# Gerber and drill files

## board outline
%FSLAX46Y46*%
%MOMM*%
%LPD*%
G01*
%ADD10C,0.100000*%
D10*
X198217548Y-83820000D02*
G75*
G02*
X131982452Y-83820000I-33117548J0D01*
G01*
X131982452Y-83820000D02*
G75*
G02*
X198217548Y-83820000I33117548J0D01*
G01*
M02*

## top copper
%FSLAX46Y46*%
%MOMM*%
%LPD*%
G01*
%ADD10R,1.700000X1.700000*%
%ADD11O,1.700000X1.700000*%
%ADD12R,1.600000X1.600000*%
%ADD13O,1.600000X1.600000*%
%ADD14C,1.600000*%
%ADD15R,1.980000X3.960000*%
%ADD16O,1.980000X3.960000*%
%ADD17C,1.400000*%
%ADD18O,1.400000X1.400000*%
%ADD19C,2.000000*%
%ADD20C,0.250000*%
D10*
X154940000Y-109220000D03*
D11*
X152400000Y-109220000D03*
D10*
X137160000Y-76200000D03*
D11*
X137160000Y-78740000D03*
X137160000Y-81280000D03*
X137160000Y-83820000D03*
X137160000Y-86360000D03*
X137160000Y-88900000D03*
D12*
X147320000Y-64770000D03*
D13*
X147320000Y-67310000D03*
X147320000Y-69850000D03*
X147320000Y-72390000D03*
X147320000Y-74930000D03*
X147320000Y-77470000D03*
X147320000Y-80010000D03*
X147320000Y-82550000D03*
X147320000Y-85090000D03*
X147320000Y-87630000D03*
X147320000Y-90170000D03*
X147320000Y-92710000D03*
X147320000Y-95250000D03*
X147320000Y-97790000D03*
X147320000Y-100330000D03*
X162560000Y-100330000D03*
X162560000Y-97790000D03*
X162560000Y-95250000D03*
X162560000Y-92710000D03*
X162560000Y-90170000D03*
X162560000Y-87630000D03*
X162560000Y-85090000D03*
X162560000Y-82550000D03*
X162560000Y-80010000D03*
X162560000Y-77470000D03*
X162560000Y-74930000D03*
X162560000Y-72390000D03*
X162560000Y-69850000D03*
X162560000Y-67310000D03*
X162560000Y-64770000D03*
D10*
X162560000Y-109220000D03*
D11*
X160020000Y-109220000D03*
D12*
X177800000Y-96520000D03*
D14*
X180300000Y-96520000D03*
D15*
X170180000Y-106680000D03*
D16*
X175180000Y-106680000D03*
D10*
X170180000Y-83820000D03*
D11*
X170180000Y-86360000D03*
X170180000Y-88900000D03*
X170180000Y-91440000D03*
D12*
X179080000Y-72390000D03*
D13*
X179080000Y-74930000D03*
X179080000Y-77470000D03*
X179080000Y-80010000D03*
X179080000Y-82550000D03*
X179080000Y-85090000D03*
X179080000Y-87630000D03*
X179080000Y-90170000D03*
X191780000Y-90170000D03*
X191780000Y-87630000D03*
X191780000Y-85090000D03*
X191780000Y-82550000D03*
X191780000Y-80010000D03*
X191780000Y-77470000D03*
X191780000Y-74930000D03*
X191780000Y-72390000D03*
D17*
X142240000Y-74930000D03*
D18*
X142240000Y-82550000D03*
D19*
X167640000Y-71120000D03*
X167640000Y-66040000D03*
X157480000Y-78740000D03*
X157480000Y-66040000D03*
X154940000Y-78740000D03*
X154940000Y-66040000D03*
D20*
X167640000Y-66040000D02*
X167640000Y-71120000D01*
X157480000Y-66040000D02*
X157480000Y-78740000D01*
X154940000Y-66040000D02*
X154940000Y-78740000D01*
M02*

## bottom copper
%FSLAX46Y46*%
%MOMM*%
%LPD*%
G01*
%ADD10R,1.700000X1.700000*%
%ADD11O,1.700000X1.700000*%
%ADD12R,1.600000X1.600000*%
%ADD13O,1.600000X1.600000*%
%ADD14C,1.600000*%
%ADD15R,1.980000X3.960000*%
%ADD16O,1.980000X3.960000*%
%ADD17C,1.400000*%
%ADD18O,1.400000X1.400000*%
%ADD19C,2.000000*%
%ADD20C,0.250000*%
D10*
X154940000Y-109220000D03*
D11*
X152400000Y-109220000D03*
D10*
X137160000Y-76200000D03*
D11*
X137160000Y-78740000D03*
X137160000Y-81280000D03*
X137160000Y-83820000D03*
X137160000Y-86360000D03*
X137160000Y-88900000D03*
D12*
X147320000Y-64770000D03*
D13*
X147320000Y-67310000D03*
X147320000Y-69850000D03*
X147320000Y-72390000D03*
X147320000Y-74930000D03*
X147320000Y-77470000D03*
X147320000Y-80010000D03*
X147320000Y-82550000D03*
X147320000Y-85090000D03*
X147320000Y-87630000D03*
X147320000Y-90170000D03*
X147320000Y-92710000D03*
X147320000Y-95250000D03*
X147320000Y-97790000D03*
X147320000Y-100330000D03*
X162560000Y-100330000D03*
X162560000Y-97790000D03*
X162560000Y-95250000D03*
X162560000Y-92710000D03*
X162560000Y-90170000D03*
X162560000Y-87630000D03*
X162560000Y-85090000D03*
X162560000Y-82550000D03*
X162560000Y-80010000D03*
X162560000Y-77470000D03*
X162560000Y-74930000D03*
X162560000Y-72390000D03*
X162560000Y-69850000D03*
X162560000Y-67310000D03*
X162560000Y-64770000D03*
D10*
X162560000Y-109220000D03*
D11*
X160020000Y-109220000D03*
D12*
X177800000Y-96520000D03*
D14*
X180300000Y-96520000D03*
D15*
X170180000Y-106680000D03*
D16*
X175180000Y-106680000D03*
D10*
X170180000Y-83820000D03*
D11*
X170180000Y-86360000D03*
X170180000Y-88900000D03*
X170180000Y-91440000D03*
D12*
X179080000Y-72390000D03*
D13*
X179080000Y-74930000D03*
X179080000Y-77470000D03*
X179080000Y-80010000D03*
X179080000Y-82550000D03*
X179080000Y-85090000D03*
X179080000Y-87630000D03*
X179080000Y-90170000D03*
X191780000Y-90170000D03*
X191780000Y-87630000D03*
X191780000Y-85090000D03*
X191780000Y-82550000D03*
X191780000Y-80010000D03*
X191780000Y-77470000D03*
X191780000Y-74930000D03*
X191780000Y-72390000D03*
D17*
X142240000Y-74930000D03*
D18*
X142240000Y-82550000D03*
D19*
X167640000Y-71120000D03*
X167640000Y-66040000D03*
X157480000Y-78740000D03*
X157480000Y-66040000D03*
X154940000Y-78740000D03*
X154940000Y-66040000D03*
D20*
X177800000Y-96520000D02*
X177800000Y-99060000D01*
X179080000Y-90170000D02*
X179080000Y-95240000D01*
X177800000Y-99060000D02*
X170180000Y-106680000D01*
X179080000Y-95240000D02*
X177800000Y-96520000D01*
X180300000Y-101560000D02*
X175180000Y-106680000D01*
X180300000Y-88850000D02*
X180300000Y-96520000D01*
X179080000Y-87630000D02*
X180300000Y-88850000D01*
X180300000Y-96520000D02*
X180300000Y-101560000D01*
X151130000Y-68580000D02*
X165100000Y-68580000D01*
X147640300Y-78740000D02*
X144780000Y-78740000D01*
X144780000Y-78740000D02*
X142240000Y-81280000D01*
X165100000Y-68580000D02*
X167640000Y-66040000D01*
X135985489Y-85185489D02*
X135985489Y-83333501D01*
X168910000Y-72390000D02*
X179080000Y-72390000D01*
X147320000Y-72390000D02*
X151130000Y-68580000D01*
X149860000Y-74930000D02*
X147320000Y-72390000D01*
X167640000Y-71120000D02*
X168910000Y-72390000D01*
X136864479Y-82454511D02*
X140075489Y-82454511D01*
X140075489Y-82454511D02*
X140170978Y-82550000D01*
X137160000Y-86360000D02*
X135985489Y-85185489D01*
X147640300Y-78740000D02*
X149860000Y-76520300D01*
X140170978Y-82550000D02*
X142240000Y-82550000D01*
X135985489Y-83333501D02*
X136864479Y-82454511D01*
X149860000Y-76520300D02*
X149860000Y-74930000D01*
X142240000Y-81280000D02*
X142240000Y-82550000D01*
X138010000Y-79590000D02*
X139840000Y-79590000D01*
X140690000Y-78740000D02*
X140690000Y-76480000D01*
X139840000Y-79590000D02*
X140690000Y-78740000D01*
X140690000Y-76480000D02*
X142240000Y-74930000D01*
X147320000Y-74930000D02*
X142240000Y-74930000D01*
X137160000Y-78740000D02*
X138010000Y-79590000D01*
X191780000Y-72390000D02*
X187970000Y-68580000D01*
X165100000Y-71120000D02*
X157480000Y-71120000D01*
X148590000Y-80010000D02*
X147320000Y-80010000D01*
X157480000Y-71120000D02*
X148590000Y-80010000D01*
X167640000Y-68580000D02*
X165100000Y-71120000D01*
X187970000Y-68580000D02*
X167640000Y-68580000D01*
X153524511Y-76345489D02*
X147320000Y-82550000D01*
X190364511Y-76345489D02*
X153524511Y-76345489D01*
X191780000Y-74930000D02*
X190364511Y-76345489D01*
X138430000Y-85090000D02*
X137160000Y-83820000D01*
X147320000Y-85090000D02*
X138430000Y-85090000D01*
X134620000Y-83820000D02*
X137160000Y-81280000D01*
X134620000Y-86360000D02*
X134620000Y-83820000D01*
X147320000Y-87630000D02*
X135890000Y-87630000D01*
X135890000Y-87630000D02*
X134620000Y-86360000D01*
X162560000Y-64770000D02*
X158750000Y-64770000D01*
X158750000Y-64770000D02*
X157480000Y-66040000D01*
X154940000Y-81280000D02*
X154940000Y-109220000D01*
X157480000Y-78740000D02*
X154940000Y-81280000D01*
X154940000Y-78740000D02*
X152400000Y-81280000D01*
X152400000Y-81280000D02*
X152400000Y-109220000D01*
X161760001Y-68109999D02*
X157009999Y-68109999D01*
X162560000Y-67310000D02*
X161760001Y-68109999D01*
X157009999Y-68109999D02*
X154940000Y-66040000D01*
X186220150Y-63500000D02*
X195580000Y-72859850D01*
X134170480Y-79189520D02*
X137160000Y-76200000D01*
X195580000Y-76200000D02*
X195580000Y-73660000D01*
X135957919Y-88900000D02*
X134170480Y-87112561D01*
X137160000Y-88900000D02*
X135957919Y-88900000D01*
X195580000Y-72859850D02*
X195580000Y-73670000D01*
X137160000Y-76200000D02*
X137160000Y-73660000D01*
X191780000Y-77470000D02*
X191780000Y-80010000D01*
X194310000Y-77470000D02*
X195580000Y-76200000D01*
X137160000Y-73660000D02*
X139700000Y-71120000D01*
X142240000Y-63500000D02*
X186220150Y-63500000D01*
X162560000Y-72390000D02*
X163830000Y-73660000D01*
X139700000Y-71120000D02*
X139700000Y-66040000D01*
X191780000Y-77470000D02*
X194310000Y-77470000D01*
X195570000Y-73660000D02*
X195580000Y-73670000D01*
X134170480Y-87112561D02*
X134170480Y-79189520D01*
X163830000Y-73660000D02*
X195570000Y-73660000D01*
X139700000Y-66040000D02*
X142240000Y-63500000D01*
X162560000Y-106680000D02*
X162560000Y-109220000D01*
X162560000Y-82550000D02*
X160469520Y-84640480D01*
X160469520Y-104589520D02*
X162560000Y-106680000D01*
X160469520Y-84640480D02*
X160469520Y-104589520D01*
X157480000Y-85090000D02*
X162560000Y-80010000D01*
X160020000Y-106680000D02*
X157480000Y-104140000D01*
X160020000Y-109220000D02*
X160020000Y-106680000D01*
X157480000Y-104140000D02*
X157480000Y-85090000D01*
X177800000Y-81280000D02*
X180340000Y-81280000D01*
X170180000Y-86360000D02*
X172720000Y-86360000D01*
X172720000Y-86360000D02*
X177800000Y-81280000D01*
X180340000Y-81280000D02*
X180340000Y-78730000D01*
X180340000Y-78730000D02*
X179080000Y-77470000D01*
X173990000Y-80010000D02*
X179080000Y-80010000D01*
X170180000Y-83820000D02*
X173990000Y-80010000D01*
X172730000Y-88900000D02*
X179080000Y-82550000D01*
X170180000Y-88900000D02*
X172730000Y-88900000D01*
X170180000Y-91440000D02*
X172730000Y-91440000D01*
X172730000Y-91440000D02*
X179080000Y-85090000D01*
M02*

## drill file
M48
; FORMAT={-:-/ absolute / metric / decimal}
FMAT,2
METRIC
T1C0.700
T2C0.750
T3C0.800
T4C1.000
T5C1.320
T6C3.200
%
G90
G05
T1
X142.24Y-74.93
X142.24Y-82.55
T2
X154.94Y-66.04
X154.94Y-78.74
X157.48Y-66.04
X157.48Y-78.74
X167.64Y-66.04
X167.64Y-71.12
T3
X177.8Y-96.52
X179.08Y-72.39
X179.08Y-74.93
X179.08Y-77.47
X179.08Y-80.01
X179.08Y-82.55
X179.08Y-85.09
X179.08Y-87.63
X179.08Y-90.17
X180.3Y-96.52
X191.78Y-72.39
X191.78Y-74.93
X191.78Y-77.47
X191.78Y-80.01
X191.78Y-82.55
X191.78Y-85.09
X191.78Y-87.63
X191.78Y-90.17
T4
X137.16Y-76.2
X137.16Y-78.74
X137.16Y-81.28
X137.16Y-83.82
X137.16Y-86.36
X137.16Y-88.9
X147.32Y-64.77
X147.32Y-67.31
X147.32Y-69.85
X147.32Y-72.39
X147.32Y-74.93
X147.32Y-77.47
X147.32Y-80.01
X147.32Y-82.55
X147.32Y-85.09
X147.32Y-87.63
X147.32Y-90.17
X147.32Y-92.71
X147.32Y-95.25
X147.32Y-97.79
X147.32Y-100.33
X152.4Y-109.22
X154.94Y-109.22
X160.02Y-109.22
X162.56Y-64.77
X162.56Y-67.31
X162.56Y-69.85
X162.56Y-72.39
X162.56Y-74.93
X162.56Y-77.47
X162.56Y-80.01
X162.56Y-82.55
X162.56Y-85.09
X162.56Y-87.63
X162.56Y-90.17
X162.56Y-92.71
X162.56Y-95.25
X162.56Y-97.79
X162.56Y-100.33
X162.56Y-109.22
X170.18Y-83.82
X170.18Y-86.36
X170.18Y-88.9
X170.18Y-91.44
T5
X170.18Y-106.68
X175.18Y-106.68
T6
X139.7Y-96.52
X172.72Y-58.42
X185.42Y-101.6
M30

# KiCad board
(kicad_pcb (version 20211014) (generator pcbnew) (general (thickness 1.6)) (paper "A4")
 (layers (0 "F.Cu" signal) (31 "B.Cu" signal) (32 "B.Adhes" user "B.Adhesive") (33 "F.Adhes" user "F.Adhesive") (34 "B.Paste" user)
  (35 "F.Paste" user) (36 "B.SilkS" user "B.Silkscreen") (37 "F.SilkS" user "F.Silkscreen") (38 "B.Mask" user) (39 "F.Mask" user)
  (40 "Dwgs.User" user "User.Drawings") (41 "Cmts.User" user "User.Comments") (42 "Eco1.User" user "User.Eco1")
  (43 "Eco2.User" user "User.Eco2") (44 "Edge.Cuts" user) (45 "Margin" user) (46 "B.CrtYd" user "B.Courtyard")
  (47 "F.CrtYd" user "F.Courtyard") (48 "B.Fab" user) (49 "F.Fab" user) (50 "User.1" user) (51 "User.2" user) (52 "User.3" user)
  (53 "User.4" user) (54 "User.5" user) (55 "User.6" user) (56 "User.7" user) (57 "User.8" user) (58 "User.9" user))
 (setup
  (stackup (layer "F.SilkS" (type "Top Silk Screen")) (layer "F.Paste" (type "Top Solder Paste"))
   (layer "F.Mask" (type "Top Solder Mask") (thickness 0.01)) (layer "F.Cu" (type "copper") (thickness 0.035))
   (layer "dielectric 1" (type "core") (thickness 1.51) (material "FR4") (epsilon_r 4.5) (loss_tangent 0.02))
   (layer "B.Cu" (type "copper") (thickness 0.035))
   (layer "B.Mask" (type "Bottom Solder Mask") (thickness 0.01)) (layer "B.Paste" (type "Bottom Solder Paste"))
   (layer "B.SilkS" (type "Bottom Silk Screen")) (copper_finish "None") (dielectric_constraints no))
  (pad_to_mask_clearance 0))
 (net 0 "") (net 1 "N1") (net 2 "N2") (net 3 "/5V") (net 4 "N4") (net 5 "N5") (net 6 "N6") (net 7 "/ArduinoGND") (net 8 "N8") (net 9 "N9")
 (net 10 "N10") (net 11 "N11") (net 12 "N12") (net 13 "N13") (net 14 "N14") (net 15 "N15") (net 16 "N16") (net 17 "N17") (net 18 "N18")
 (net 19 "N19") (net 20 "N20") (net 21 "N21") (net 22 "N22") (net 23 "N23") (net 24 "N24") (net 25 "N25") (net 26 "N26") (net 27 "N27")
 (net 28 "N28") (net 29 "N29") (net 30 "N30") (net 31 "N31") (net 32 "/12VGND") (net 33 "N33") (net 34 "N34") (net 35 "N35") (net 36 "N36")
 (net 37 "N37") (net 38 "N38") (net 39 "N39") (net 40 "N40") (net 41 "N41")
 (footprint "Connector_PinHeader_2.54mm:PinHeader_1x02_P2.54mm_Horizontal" (layer "F.Cu") (at 154.94 109.22 -90)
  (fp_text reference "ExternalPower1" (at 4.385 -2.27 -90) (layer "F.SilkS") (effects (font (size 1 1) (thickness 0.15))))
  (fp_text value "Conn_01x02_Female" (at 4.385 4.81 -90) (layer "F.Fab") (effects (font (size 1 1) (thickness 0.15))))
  (pad "1" thru_hole rect (at 0 0 270) (size 1.7 1.7) (drill 1) (layers *.Cu *.Mask) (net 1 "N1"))
  (pad "2" thru_hole oval (at 0 2.54 270) (size 1.7 1.7) (drill 1) (layers *.Cu *.Mask) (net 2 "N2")))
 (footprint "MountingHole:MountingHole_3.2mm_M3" (layer "F.Cu") (at 139.7 96.52)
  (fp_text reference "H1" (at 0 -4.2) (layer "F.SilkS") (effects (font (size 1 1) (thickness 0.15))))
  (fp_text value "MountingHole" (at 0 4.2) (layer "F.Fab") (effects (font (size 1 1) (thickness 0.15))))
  (pad "" np_thru_hole circle (at 0 0) (size 3.2 3.2) (drill 3.2) (layers *.Cu *.Mask)))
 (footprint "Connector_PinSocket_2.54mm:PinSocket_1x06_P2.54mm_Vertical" (layer "F.Cu") (at 137.16 76.2)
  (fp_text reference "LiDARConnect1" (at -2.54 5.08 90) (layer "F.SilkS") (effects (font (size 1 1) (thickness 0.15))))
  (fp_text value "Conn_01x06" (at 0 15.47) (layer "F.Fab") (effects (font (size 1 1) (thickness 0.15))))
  (pad "1" thru_hole rect (at 0 0) (size 1.7 1.7) (drill 1) (layers *.Cu *.Mask) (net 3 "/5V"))
  (pad "2" thru_hole oval (at 0 2.54) (size 1.7 1.7) (drill 1) (layers *.Cu *.Mask) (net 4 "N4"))
  (pad "3" thru_hole oval (at 0 5.08) (size 1.7 1.7) (drill 1) (layers *.Cu *.Mask) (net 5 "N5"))
  (pad "4" thru_hole oval (at 0 7.62) (size 1.7 1.7) (drill 1) (layers *.Cu *.Mask) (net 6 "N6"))
  (pad "5" thru_hole oval (at 0 10.16) (size 1.7 1.7) (drill 1) (layers *.Cu *.Mask) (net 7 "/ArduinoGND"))
  (pad "6" thru_hole oval (at 0 12.7) (size 1.7 1.7) (drill 1) (layers *.Cu *.Mask) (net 3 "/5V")))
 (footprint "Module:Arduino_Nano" (layer "F.Cu") (at 147.32 64.77)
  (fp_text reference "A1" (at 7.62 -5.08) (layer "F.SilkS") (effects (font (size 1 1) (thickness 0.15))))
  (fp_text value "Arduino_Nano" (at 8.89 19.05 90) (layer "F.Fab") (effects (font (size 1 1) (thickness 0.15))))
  (pad "1" thru_hole rect (at 0 0) (size 1.6 1.6) (drill 1) (layers *.Cu *.Mask) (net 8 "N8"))
  (pad "2" thru_hole oval (at 0 2.54) (size 1.6 1.6) (drill 1) (layers *.Cu *.Mask) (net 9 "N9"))
  (pad "3" thru_hole oval (at 0 5.08) (size 1.6 1.6) (drill 1) (layers *.Cu *.Mask) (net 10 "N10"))
  (pad "4" thru_hole oval (at 0 7.62) (size 1.6 1.6) (drill 1) (layers *.Cu *.Mask) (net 7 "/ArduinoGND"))
  (pad "5" thru_hole oval (at 0 10.16) (size 1.6 1.6) (drill 1) (layers *.Cu *.Mask) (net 4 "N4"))
  (pad "6" thru_hole oval (at 0 12.7) (size 1.6 1.6) (drill 1) (layers *.Cu *.Mask) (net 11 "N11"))
  (pad "7" thru_hole oval (at 0 15.24) (size 1.6 1.6) (drill 1) (layers *.Cu *.Mask) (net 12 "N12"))
  (pad "8" thru_hole oval (at 0 17.78) (size 1.6 1.6) (drill 1) (layers *.Cu *.Mask) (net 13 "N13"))
  (pad "9" thru_hole oval (at 0 20.32) (size 1.6 1.6) (drill 1) (layers *.Cu *.Mask) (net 6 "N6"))
  (pad "10" thru_hole oval (at 0 22.86) (size 1.6 1.6) (drill 1) (layers *.Cu *.Mask) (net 5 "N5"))
  (pad "11" thru_hole oval (at 0 25.4) (size 1.6 1.6) (drill 1) (layers *.Cu *.Mask) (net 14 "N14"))
  (pad "12" thru_hole oval (at 0 27.94) (size 1.6 1.6) (drill 1) (layers *.Cu *.Mask) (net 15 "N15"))
  (pad "13" thru_hole oval (at 0 30.48) (size 1.6 1.6) (drill 1) (layers *.Cu *.Mask) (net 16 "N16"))
  (pad "14" thru_hole oval (at 0 33.02) (size 1.6 1.6) (drill 1) (layers *.Cu *.Mask) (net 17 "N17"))
  (pad "15" thru_hole oval (at 0 35.56) (size 1.6 1.6) (drill 1) (layers *.Cu *.Mask) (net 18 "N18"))
  (pad "16" thru_hole oval (at 15.24 35.56) (size 1.6 1.6) (drill 1) (layers *.Cu *.Mask) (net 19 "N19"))
  (pad "17" thru_hole oval (at 15.24 33.02) (size 1.6 1.6) (drill 1) (layers *.Cu *.Mask) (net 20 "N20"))
  (pad "18" thru_hole oval (at 15.24 30.48) (size 1.6 1.6) (drill 1) (layers *.Cu *.Mask) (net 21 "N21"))
  (pad "19" thru_hole oval (at 15.24 27.94) (size 1.6 1.6) (drill 1) (layers *.Cu *.Mask) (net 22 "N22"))
  (pad "20" thru_hole oval (at 15.24 25.4) (size 1.6 1.6) (drill 1) (layers *.Cu *.Mask) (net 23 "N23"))
  (pad "21" thru_hole oval (at 15.24 22.86) (size 1.6 1.6) (drill 1) (layers *.Cu *.Mask) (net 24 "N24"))
  (pad "22" thru_hole oval (at 15.24 20.32) (size 1.6 1.6) (drill 1) (layers *.Cu *.Mask) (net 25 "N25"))
  (pad "23" thru_hole oval (at 15.24 17.78) (size 1.6 1.6) (drill 1) (layers *.Cu *.Mask) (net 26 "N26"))
  (pad "24" thru_hole oval (at 15.24 15.24) (size 1.6 1.6) (drill 1) (layers *.Cu *.Mask) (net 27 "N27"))
  (pad "25" thru_hole oval (at 15.24 12.7) (size 1.6 1.6) (drill 1) (layers *.Cu *.Mask) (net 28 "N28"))
  (pad "26" thru_hole oval (at 15.24 10.16) (size 1.6 1.6) (drill 1) (layers *.Cu *.Mask) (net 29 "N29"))
  (pad "27" thru_hole oval (at 15.24 7.62) (size 1.6 1.6) (drill 1) (layers *.Cu *.Mask) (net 3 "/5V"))
  (pad "28" thru_hole oval (at 15.24 5.08) (size 1.6 1.6) (drill 1) (layers *.Cu *.Mask) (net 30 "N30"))
  (pad "29" thru_hole oval (at 15.24 2.54) (size 1.6 1.6) (drill 1) (layers *.Cu *.Mask) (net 2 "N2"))
  (pad "30" thru_hole oval (at 15.24 0) (size 1.6 1.6) (drill 1) (layers *.Cu *.Mask) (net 1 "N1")))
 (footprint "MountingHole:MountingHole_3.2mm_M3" (layer "F.Cu") (at 185.42 101.6)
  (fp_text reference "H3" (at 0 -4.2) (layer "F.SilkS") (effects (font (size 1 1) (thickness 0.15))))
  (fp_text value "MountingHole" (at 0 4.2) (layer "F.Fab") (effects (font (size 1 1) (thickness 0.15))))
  (pad "" np_thru_hole circle (at 0 0) (size 3.2 3.2) (drill 3.2) (layers *.Cu *.Mask)))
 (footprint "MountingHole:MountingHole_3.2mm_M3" (layer "F.Cu") (at 172.72 58.42)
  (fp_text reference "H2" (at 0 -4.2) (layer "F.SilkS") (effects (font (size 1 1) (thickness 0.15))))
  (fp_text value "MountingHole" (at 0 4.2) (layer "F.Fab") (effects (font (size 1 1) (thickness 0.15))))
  (pad "" np_thru_hole circle (at 0 0) (size 3.2 3.2) (drill 3.2) (layers *.Cu *.Mask)))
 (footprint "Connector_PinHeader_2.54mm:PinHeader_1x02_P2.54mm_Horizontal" (layer "F.Cu") (at 162.56 109.22 -90)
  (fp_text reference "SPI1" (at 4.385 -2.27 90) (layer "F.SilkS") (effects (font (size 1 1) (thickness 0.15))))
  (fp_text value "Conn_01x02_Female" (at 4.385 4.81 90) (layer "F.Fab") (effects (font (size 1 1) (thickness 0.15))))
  (pad "1" thru_hole rect (at 0 0 270) (size 1.7 1.7) (drill 1) (layers *.Cu *.Mask) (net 26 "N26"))
  (pad "2" thru_hole oval (at 0 2.54 270) (size 1.7 1.7) (drill 1) (layers *.Cu *.Mask) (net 27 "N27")))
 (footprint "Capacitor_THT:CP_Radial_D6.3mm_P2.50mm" (layer "F.Cu") (at 177.8 96.52)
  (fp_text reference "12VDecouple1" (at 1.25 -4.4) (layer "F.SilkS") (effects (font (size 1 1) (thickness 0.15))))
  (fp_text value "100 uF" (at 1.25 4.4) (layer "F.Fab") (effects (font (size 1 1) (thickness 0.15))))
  (pad "1" thru_hole rect (at 0 0) (size 1.6 1.6) (drill 0.8) (layers *.Cu *.Mask) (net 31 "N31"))
  (pad "2" thru_hole circle (at 2.5 0) (size 1.6 1.6) (drill 0.8) (layers *.Cu *.Mask) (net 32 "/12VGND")))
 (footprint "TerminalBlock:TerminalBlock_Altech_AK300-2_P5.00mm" (layer "F.Cu") (at 170.18 106.68)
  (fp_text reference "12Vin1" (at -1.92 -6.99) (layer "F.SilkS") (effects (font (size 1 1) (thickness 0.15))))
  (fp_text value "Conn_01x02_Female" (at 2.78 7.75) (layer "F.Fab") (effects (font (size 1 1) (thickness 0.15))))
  (pad "1" thru_hole rect (at 0 0) (size 1.98 3.96) (drill 1.32) (layers *.Cu *.Mask) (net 31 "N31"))
  (pad "2" thru_hole oval (at 5 0) (size 1.98 3.96) (drill 1.32) (layers *.Cu *.Mask) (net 32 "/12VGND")))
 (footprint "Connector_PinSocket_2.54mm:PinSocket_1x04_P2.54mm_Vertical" (layer "F.Cu") (at 170.18 83.82)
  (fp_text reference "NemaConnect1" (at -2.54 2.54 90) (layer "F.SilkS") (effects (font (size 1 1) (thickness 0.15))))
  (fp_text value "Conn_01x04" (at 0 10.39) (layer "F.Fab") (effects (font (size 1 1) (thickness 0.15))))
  (pad "1" thru_hole rect (at 0 0) (size 1.7 1.7) (drill 1) (layers *.Cu *.Mask) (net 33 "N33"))
  (pad "2" thru_hole oval (at 0 2.54) (size 1.7 1.7) (drill 1) (layers *.Cu *.Mask) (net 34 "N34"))
  (pad "3" thru_hole oval (at 0 5.08) (size 1.7 1.7) (drill 1) (layers *.Cu *.Mask) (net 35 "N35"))
  (pad "4" thru_hole oval (at 0 7.62) (size 1.7 1.7) (drill 1) (layers *.Cu *.Mask) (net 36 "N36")))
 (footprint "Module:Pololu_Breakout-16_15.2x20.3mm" (layer "F.Cu") (at 179.08 72.39)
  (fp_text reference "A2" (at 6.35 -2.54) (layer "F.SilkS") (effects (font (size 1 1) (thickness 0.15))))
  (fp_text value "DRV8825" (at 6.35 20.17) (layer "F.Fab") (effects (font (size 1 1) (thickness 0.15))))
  (pad "1" thru_hole rect (at 0 0) (size 1.6 1.6) (drill 0.8) (layers *.Cu *.Mask) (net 7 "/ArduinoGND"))
  (pad "2" thru_hole oval (at 0 2.54) (size 1.6 1.6) (drill 0.8) (layers *.Cu *.Mask) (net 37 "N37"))
  (pad "3" thru_hole oval (at 0 5.08) (size 1.6 1.6) (drill 0.8) (layers *.Cu *.Mask) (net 34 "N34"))
  (pad "4" thru_hole oval (at 0 7.62) (size 1.6 1.6) (drill 0.8) (layers *.Cu *.Mask) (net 33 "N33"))
  (pad "5" thru_hole oval (at 0 10.16) (size 1.6 1.6) (drill 0.8) (layers *.Cu *.Mask) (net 35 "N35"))
  (pad "6" thru_hole oval (at 0 12.7) (size 1.6 1.6) (drill 0.8) (layers *.Cu *.Mask) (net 36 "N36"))
  (pad "7" thru_hole oval (at 0 15.24) (size 1.6 1.6) (drill 0.8) (layers *.Cu *.Mask) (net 32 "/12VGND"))
  (pad "8" thru_hole oval (at 0 17.78) (size 1.6 1.6) (drill 0.8) (layers *.Cu *.Mask) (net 31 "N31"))
  (pad "9" thru_hole oval (at 12.7 17.78) (size 1.6 1.6) (drill 0.8) (layers *.Cu *.Mask) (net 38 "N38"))
  (pad "10" thru_hole oval (at 12.7 15.24) (size 1.6 1.6) (drill 0.8) (layers *.Cu *.Mask) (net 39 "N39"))
  (pad "11" thru_hole oval (at 12.7 12.7) (size 1.6 1.6) (drill 0.8) (layers *.Cu *.Mask) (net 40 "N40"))
  (pad "12" thru_hole oval (at 12.7 10.16) (size 1.6 1.6) (drill 0.8) (layers *.Cu *.Mask) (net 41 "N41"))
  (pad "13" thru_hole oval (at 12.7 7.62) (size 1.6 1.6) (drill 0.8) (layers *.Cu *.Mask) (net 3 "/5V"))
  (pad "14" thru_hole oval (at 12.7 5.08) (size 1.6 1.6) (drill 0.8) (layers *.Cu *.Mask) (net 3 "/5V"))
  (pad "15" thru_hole oval (at 12.7 2.54) (size 1.6 1.6) (drill 0.8) (layers *.Cu *.Mask) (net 13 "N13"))
  (pad "16" thru_hole oval (at 12.7 0) (size 1.6 1.6) (drill 0.8) (layers *.Cu *.Mask) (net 12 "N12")))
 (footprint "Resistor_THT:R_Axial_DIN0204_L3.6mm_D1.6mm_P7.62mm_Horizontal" (layer "B.Cu") (at 142.24 74.93 -90)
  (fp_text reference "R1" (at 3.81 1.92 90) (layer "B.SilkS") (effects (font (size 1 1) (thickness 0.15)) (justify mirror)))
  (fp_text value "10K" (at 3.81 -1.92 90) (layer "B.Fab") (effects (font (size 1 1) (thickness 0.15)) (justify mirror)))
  (pad "1" thru_hole circle (at 0 0 270) (size 1.4 1.4) (drill 0.7) (layers *.Cu *.Mask) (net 4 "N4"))
  (pad "2" thru_hole oval (at 7.62 0 270) (size 1.4 1.4) (drill 0.7) (layers *.Cu *.Mask) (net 7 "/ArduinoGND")))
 (gr_circle (center 165.1 83.82) (end 193.04 66.04) (layer "Edge.Cuts") (width 0.1) (fill none))
 (segment (start 177.8 96.52) (end 177.8 99.06) (width 0.25) (layer "B.Cu") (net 31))
 (segment (start 179.08 90.17) (end 179.08 95.24) (width 0.25) (layer "B.Cu") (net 31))
 (segment (start 177.8 99.06) (end 170.18 106.68) (width 0.25) (layer "B.Cu") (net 31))
 (segment (start 179.08 95.24) (end 177.8 96.52) (width 0.25) (layer "B.Cu") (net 31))
 (segment (start 180.3 101.56) (end 175.18 106.68) (width 0.25) (layer "B.Cu") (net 32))
 (segment (start 180.3 88.85) (end 180.3 96.52) (width 0.25) (layer "B.Cu") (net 32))
 (segment (start 179.08 87.63) (end 180.3 88.85) (width 0.25) (layer "B.Cu") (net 32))
 (segment (start 180.3 96.52) (end 180.3 101.56) (width 0.25) (layer "B.Cu") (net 32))
 (segment (start 167.64 66.04) (end 167.64 71.12) (width 0.25) (layer "F.Cu") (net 7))
 (via (at 167.64 71.12) (size 2) (drill 0.75) (layers "F.Cu" "B.Cu") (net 7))
 (via (at 167.64 66.04) (size 2) (drill 0.75) (layers "F.Cu" "B.Cu") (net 7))
 (segment (start 151.13 68.58) (end 165.1 68.58) (width 0.25) (layer "B.Cu") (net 7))
 (segment (start 147.6403 78.74) (end 144.78 78.74) (width 0.25) (layer "B.Cu") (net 7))
 (segment (start 144.78 78.74) (end 142.24 81.28) (width 0.25) (layer "B.Cu") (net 7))
 (segment (start 165.1 68.58) (end 167.64 66.04) (width 0.25) (layer "B.Cu") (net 7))
 (segment (start 135.985489 85.185489) (end 135.985489 83.333501) (width 0.25) (layer "B.Cu") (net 7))
 (segment (start 168.91 72.39) (end 179.08 72.39) (width 0.25) (layer "B.Cu") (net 7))
 (segment (start 147.32 72.39) (end 151.13 68.58) (width 0.25) (layer "B.Cu") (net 7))
 (segment (start 149.86 74.93) (end 147.32 72.39) (width 0.25) (layer "B.Cu") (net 7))
 (segment (start 167.64 71.12) (end 168.91 72.39) (width 0.25) (layer "B.Cu") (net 7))
 (segment (start 136.864479 82.454511) (end 140.075489 82.454511) (width 0.25) (layer "B.Cu") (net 7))
 (segment (start 140.075489 82.454511) (end 140.170978 82.55) (width 0.25) (layer "B.Cu") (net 7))
 (segment (start 137.16 86.36) (end 135.985489 85.185489) (width 0.25) (layer "B.Cu") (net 7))
 (segment (start 147.6403 78.74) (end 149.86 76.5203) (width 0.25) (layer "B.Cu") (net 7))
 (segment (start 140.170978 82.55) (end 142.24 82.55) (width 0.25) (layer "B.Cu") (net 7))
 (segment (start 135.985489 83.333501) (end 136.864479 82.454511) (width 0.25) (layer "B.Cu") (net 7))
 (segment (start 149.86 76.5203) (end 149.86 74.93) (width 0.25) (layer "B.Cu") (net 7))
 (segment (start 142.24 81.28) (end 142.24 82.55) (width 0.25) (layer "B.Cu") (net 7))
 (segment (start 138.01 79.59) (end 139.84 79.59) (width 0.25) (layer "B.Cu") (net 4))
 (segment (start 140.69 78.74) (end 140.69 76.48) (width 0.25) (layer "B.Cu") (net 4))
 (segment (start 139.84 79.59) (end 140.69 78.74) (width 0.25) (layer "B.Cu") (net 4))
 (segment (start 140.69 76.48) (end 142.24 74.93) (width 0.25) (layer "B.Cu") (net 4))
 (segment (start 147.32 74.93) (end 142.24 74.93) (width 0.25) (layer "B.Cu") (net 4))
 (segment (start 137.16 78.74) (end 138.01 79.59) (width 0.25) (layer "B.Cu") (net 4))
 (segment (start 191.78 72.39) (end 187.97 68.58) (width 0.25) (layer "B.Cu") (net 12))
 (segment (start 165.1 71.12) (end 157.48 71.12) (width 0.25) (layer "B.Cu") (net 12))
 (segment (start 148.59 80.01) (end 147.32 80.01) (width 0.25) (layer "B.Cu") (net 12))
 (segment (start 157.48 71.12) (end 148.59 80.01) (width 0.25) (layer "B.Cu") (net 12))
 (segment (start 167.64 68.58) (end 165.1 71.12) (width 0.25) (layer "B.Cu") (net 12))
 (segment (start 187.97 68.58) (end 167.64 68.58) (width 0.25) (layer "B.Cu") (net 12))
 (segment (start 153.524511 76.345489) (end 147.32 82.55) (width 0.25) (layer "B.Cu") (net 13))
 (segment (start 190.364511 76.345489) (end 153.524511 76.345489) (width 0.25) (layer "B.Cu") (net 13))
 (segment (start 191.78 74.93) (end 190.364511 76.345489) (width 0.25) (layer "B.Cu") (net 13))
 (segment (start 138.43 85.09) (end 137.16 83.82) (width 0.25) (layer "B.Cu") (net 6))
 (segment (start 147.32 85.09) (end 138.43 85.09) (width 0.25) (layer "B.Cu") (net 6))
 (segment (start 134.62 83.82) (end 137.16 81.28) (width 0.25) (layer "B.Cu") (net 5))
 (segment (start 134.62 86.36) (end 134.62 83.82) (width 0.25) (layer "B.Cu") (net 5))
 (segment (start 147.32 87.63) (end 135.89 87.63) (width 0.25) (layer "B.Cu") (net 5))
 (segment (start 135.89 87.63) (end 134.62 86.36) (width 0.25) (layer "B.Cu") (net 5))
 (segment (start 157.48 66.04) (end 157.48 78.74) (width 0.25) (layer "F.Cu") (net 1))
 (via (at 157.48 78.74) (size 2) (drill 0.75) (layers "F.Cu" "B.Cu") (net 1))
 (via (at 157.48 66.04) (size 2) (drill 0.75) (layers "F.Cu" "B.Cu") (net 1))
 (segment (start 162.56 64.77) (end 158.75 64.77) (width 0.25) (layer "B.Cu") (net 1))
 (segment (start 158.75 64.77) (end 157.48 66.04) (width 0.25) (layer "B.Cu") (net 1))
 (segment (start 154.94 81.28) (end 154.94 109.22) (width 0.25) (layer "B.Cu") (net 1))
 (segment (start 157.48 78.74) (end 154.94 81.28) (width 0.25) (layer "B.Cu") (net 1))
 (segment (start 154.94 66.04) (end 154.94 78.74) (width 0.25) (layer "F.Cu") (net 2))
 (via (at 154.94 78.74) (size 2) (drill 0.75) (layers "F.Cu" "B.Cu") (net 2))
 (via (at 154.94 66.04) (size 2) (drill 0.75) (layers "F.Cu" "B.Cu") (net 2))
 (segment (start 154.94 78.74) (end 152.4 81.28) (width 0.25) (layer "B.Cu") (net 2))
 (segment (start 152.4 81.28) (end 152.4 109.22) (width 0.25) (layer "B.Cu") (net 2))
 (segment (start 161.760001 68.109999) (end 157.009999 68.109999) (width 0.25) (layer "B.Cu") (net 2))
 (segment (start 162.56 67.31) (end 161.760001 68.109999) (width 0.25) (layer "B.Cu") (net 2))
 (segment (start 157.009999 68.109999) (end 154.94 66.04) (width 0.25) (layer "B.Cu") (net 2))
 (segment (start 186.22015 63.5) (end 195.58 72.85985) (width 0.25) (layer "B.Cu") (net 3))
 (segment (start 134.17048 79.18952) (end 137.16 76.2) (width 0.25) (layer "B.Cu") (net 3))
 (segment (start 195.58 76.2) (end 195.58 73.66) (width 0.25) (layer "B.Cu") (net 3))
 (segment (start 135.957919 88.9) (end 134.17048 87.112561) (width 0.25) (layer "B.Cu") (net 3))
 (segment (start 137.16 88.9) (end 135.957919 88.9) (width 0.25) (layer "B.Cu") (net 3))
 (segment (start 195.58 72.85985) (end 195.58 73.67) (width 0.25) (layer "B.Cu") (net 3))
 (segment (start 137.16 76.2) (end 137.16 73.66) (width 0.25) (layer "B.Cu") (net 3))
 (segment (start 191.78 77.47) (end 191.78 80.01) (width 0.25) (layer "B.Cu") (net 3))
 (segment (start 194.31 77.47) (end 195.58 76.2) (width 0.25) (layer "B.Cu") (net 3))
 (segment (start 137.16 73.66) (end 139.7 71.12) (width 0.25) (layer "B.Cu") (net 3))
 (segment (start 142.24 63.5) (end 186.22015 63.5) (width 0.25) (layer "B.Cu") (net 3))
 (segment (start 162.56 72.39) (end 163.83 73.66) (width 0.25) (layer "B.Cu") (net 3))
 (segment (start 139.7 71.12) (end 139.7 66.04) (width 0.25) (layer "B.Cu") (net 3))
 (segment (start 191.78 77.47) (end 194.31 77.47) (width 0.25) (layer "B.Cu") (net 3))
 (segment (start 195.57 73.66) (end 195.58 73.67) (width 0.25) (layer "B.Cu") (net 3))
 (segment (start 134.17048 87.112561) (end 134.17048 79.18952) (width 0.25) (layer "B.Cu") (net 3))
 (segment (start 163.83 73.66) (end 195.57 73.66) (width 0.25) (layer "B.Cu") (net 3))
 (segment (start 139.7 66.04) (end 142.24 63.5) (width 0.25) (layer "B.Cu") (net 3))
 (segment (start 162.56 106.68) (end 162.56 109.22) (width 0.25) (layer "B.Cu") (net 26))
 (segment (start 162.56 82.55) (end 160.46952 84.64048) (width 0.25) (layer "B.Cu") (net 26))
 (segment (start 160.46952 104.58952) (end 162.56 106.68) (width 0.25) (layer "B.Cu") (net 26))
 (segment (start 160.46952 84.64048) (end 160.46952 104.58952) (width 0.25) (layer "B.Cu") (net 26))
 (segment (start 157.48 85.09) (end 162.56 80.01) (width 0.25) (layer "B.Cu") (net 27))
 (segment (start 160.02 106.68) (end 157.48 104.14) (width 0.25) (layer "B.Cu") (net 27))
 (segment (start 160.02 109.22) (end 160.02 106.68) (width 0.25) (layer "B.Cu") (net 27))
 (segment (start 157.48 104.14) (end 157.48 85.09) (width 0.25) (layer "B.Cu") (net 27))
 (segment (start 177.8 81.28) (end 180.34 81.28) (width 0.25) (layer "B.Cu") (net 34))
 (segment (start 170.18 86.36) (end 172.72 86.36) (width 0.25) (layer "B.Cu") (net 34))
 (segment (start 172.72 86.36) (end 177.8 81.28) (width 0.25) (layer "B.Cu") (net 34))
 (segment (start 180.34 81.28) (end 180.34 78.73) (width 0.25) (layer "B.Cu") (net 34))
 (segment (start 180.34 78.73) (end 179.08 77.47) (width 0.25) (layer "B.Cu") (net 34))
 (segment (start 173.99 80.01) (end 179.08 80.01) (width 0.25) (layer "B.Cu") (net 33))
 (segment (start 170.18 83.82) (end 173.99 80.01) (width 0.25) (layer "B.Cu") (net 33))
 (segment (start 172.73 88.9) (end 179.08 82.55) (width 0.25) (layer "B.Cu") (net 35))
 (segment (start 170.18 88.9) (end 172.73 88.9) (width 0.25) (layer "B.Cu") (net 35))
 (segment (start 170.18 91.44) (end 172.73 91.44) (width 0.25) (layer "B.Cu") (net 36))
 (segment (start 172.73 91.44) (end 179.08 85.09) (width 0.25) (layer "B.Cu") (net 36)))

